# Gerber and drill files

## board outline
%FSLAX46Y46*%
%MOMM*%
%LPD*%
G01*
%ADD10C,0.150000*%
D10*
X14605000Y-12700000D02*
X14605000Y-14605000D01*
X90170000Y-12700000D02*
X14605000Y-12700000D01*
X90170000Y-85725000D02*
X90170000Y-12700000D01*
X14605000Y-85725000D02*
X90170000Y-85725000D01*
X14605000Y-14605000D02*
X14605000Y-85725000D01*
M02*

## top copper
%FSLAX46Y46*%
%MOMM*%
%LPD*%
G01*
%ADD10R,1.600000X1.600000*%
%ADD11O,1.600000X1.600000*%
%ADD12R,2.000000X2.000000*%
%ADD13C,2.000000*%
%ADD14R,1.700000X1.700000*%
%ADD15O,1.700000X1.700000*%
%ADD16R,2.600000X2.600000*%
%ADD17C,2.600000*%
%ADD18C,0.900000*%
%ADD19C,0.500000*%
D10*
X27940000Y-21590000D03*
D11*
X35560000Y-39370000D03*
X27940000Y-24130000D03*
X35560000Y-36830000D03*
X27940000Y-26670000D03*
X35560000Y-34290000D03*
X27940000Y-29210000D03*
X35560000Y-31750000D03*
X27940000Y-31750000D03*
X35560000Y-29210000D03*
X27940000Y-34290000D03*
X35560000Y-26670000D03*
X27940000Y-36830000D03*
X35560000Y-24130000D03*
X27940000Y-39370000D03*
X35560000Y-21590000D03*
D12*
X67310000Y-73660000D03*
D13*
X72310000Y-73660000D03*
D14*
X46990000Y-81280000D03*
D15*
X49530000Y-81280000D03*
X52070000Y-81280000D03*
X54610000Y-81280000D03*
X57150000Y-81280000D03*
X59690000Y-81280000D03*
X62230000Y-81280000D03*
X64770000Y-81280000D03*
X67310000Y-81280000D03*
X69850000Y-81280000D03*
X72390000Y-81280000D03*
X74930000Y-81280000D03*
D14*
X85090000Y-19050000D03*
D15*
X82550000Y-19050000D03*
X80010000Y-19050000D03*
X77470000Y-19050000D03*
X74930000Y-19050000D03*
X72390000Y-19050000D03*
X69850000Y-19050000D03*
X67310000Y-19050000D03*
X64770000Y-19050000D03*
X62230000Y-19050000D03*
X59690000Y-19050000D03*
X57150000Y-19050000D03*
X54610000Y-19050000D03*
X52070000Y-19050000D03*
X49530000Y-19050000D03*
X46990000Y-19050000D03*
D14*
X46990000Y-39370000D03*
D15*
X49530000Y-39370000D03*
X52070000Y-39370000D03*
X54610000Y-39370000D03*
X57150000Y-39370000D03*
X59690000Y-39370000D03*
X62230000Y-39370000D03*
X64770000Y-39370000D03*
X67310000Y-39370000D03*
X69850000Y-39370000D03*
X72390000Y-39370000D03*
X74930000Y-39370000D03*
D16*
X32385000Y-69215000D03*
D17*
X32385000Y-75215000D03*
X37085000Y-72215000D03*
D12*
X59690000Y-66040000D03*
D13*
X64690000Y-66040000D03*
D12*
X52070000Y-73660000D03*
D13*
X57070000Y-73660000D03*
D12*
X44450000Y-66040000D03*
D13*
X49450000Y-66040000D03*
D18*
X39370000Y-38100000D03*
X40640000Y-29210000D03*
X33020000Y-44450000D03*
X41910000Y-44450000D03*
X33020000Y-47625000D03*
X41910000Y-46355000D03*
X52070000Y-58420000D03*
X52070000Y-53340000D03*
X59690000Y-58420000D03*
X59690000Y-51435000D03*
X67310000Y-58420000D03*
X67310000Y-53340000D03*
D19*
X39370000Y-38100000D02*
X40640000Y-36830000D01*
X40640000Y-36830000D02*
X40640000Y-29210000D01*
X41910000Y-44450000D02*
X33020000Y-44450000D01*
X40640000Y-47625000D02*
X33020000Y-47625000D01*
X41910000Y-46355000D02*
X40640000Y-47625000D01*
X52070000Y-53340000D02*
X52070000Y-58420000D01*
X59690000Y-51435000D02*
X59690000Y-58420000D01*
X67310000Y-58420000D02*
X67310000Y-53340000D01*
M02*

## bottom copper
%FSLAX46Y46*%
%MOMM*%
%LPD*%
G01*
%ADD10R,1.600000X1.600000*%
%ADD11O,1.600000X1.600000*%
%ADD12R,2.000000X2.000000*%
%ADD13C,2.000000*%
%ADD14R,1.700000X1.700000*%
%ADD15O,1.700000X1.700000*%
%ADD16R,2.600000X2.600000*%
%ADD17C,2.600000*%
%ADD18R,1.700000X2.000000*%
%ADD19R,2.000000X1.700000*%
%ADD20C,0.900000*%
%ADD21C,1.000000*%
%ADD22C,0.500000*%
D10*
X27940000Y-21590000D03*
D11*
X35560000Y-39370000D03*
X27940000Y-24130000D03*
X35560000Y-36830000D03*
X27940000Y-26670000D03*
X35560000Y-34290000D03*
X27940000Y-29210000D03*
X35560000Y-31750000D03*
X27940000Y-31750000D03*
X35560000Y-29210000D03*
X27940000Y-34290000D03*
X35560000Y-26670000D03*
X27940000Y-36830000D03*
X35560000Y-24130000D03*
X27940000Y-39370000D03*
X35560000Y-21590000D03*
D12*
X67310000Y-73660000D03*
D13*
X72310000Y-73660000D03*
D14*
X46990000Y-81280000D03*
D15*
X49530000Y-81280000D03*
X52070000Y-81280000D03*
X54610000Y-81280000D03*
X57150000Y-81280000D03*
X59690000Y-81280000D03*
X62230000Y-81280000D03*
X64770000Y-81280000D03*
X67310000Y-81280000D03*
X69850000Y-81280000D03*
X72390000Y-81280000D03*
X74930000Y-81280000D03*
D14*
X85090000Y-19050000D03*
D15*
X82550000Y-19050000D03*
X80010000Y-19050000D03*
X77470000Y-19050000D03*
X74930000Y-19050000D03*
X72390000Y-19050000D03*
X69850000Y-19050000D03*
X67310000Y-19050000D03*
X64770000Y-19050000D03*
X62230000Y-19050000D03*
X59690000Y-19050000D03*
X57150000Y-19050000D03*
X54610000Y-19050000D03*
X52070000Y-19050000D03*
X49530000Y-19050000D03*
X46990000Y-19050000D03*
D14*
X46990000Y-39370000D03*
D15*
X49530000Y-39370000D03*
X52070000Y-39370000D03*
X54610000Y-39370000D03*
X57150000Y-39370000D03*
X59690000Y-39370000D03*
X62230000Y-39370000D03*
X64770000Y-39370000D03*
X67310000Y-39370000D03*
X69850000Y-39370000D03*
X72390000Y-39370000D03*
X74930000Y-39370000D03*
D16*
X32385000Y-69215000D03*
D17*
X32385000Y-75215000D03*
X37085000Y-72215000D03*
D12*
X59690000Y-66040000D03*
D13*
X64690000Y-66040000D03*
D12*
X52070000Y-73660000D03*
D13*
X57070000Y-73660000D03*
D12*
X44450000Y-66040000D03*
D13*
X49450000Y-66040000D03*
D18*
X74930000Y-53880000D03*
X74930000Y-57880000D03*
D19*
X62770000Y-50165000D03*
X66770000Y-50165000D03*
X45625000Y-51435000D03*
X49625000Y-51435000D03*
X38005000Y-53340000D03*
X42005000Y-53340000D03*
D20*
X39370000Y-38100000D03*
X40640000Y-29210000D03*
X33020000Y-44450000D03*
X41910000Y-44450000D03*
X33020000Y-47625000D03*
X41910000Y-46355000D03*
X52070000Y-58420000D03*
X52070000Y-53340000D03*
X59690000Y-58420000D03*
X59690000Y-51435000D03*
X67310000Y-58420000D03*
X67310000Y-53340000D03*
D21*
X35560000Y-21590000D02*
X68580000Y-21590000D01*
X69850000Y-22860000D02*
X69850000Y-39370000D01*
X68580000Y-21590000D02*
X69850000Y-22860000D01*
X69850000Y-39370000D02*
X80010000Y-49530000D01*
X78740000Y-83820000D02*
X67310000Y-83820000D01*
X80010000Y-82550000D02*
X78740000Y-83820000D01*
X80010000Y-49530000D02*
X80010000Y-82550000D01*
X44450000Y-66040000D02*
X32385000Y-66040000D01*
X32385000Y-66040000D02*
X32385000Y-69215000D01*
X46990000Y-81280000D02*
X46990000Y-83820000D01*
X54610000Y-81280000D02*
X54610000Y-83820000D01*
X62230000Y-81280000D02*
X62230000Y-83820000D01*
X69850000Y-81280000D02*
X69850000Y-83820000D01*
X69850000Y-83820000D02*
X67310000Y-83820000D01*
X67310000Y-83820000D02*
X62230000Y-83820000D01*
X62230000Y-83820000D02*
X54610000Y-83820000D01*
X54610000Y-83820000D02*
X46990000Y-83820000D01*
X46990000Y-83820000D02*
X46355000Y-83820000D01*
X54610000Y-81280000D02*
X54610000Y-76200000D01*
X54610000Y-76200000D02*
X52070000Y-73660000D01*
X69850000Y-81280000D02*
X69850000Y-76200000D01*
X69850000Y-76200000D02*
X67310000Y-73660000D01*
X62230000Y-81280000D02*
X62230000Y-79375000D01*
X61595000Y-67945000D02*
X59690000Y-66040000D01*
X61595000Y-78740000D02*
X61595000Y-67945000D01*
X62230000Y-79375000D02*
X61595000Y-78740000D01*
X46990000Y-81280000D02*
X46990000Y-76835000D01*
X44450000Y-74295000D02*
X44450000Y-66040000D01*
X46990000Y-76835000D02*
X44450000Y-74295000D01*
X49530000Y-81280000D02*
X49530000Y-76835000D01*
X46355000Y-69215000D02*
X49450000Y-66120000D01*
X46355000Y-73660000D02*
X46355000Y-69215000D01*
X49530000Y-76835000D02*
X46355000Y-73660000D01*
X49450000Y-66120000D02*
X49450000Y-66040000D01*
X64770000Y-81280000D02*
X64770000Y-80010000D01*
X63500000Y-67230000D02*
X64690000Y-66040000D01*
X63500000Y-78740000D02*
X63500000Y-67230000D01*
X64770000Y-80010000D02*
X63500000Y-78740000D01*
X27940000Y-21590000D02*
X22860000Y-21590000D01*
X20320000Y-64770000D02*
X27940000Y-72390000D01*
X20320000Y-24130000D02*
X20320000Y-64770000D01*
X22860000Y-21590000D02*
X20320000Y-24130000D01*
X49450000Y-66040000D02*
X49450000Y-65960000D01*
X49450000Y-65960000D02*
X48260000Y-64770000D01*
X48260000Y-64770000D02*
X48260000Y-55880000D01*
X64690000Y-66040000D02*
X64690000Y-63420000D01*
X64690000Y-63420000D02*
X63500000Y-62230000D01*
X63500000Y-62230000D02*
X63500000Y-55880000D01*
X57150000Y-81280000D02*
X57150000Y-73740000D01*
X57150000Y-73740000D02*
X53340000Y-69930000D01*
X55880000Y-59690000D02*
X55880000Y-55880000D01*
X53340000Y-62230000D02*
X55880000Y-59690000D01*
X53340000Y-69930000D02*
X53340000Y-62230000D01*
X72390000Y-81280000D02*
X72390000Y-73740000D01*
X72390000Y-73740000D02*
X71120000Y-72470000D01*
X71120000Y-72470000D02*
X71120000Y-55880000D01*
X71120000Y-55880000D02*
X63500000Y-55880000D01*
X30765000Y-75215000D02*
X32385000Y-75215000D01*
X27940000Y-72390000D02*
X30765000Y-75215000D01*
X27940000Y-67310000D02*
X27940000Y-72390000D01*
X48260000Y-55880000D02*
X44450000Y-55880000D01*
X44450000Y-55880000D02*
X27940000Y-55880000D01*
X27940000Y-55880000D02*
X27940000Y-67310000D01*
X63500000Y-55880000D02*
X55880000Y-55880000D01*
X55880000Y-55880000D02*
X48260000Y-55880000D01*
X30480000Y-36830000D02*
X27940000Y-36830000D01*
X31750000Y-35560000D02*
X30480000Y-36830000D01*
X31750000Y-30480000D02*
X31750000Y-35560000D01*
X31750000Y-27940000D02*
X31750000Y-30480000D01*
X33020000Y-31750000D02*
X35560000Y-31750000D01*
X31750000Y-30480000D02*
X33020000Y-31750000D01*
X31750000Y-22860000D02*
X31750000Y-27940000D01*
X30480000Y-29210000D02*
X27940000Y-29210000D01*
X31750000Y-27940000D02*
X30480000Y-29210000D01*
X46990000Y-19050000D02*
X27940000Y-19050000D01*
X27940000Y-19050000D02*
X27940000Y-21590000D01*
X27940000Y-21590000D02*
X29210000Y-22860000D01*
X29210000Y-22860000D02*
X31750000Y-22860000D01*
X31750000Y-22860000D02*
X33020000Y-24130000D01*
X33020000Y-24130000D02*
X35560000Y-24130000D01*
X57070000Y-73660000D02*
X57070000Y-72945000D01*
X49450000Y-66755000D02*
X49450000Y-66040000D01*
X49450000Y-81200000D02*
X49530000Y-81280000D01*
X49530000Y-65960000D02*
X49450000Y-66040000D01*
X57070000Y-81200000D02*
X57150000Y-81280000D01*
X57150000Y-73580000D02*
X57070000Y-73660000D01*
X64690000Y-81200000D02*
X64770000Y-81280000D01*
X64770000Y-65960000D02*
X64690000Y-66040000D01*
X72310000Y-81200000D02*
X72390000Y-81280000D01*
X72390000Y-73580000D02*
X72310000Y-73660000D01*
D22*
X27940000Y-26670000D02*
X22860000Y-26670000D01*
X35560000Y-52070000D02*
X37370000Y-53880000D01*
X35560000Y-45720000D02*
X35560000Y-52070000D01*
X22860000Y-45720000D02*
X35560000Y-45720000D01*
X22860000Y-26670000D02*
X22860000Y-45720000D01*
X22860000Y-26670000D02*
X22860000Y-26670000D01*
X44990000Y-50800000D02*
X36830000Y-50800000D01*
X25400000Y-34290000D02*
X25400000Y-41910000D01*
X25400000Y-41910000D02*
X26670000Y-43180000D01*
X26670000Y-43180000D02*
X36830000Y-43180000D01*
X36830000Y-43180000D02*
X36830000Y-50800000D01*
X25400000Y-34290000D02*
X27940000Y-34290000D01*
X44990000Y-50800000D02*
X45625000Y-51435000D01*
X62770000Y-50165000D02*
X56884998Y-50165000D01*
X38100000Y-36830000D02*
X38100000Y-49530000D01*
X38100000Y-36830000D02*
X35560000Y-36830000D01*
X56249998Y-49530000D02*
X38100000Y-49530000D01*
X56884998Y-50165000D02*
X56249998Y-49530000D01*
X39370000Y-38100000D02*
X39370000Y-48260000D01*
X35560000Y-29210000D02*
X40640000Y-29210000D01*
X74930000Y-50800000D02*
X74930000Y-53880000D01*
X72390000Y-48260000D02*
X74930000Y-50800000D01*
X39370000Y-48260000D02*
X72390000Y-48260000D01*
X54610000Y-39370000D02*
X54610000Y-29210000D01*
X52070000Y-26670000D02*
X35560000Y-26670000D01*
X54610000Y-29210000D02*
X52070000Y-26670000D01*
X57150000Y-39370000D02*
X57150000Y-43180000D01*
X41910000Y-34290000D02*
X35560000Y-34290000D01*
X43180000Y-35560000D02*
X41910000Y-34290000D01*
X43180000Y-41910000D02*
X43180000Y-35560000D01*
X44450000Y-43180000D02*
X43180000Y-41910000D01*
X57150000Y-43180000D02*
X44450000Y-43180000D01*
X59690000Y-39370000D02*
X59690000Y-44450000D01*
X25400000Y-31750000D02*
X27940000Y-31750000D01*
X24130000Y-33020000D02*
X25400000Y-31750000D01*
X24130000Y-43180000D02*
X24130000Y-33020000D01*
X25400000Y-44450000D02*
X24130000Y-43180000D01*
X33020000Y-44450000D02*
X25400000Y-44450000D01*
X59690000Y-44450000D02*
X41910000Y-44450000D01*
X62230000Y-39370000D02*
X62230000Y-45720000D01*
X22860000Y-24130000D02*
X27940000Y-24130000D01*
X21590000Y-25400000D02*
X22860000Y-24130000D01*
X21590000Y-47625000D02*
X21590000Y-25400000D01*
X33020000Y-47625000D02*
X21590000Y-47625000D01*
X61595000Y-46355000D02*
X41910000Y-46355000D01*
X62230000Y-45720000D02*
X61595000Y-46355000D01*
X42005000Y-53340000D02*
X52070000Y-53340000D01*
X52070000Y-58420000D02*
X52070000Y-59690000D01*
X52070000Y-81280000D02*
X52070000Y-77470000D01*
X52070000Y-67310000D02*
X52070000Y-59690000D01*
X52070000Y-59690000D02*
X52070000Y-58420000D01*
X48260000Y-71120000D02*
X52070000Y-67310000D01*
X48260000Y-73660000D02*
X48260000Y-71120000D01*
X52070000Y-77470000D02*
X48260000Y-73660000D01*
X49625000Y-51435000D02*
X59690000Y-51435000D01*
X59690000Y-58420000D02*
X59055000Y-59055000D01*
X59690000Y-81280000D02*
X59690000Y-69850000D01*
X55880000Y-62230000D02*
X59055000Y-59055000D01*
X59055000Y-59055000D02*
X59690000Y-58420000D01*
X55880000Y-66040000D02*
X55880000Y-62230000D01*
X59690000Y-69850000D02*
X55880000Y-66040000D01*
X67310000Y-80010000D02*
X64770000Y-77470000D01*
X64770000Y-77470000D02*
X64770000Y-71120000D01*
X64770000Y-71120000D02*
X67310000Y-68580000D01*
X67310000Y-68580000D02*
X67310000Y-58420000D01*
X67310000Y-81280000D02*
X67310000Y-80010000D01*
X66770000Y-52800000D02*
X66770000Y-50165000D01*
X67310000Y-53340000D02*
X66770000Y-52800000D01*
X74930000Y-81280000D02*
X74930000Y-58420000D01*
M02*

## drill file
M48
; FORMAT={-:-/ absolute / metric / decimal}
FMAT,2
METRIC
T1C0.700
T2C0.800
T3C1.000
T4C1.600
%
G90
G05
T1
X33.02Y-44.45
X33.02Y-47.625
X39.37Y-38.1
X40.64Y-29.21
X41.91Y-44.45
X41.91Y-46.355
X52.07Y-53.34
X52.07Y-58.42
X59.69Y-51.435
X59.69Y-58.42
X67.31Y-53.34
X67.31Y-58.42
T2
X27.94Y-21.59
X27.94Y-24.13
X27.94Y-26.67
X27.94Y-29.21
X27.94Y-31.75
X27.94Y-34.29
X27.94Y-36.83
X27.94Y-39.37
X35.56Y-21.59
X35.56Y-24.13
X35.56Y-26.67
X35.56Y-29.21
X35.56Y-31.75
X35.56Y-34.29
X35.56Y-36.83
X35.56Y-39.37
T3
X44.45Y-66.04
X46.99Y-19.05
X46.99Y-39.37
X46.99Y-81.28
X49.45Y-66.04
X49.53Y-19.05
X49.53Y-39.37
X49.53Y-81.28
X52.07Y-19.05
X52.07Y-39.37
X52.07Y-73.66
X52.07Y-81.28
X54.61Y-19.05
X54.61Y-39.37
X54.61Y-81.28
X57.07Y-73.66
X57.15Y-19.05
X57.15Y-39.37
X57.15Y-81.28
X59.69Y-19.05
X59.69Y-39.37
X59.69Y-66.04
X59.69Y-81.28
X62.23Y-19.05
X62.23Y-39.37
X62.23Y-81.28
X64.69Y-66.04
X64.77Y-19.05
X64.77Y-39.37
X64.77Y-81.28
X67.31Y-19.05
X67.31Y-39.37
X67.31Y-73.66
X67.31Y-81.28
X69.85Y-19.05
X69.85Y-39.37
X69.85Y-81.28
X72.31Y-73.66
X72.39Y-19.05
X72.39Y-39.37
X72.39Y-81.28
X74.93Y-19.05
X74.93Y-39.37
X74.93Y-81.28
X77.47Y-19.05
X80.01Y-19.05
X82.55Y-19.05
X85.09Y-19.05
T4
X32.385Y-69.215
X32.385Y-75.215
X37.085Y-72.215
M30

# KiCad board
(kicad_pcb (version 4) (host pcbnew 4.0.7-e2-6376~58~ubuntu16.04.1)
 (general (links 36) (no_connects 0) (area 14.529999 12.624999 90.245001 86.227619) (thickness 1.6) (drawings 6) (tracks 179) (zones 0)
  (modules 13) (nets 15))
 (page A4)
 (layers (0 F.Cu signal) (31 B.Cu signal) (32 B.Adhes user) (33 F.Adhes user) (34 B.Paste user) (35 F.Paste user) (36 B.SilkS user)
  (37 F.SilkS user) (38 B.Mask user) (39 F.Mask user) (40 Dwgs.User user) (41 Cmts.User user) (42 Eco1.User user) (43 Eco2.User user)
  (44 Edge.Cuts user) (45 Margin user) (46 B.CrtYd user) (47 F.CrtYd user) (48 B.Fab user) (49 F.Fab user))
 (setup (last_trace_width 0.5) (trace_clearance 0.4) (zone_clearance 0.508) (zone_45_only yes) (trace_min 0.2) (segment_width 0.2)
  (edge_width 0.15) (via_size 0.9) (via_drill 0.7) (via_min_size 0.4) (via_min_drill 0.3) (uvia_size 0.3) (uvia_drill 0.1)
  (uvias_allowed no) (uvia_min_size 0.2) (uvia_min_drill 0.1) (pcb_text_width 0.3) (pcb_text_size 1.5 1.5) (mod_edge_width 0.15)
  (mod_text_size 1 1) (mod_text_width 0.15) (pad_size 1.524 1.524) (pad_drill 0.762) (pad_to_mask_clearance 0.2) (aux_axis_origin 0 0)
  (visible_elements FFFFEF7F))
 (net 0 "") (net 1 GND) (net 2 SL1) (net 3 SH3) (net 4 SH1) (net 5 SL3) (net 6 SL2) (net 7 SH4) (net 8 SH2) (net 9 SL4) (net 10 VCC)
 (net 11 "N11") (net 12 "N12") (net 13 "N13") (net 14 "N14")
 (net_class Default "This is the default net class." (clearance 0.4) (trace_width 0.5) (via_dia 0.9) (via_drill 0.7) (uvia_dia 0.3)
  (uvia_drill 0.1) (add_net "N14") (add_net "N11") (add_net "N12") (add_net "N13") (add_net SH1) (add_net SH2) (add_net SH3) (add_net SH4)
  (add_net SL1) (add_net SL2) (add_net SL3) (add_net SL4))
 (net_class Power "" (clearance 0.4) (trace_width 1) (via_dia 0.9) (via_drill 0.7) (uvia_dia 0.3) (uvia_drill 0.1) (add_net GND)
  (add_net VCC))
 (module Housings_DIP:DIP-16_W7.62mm (layer F.Cu) (at 27.94 21.59)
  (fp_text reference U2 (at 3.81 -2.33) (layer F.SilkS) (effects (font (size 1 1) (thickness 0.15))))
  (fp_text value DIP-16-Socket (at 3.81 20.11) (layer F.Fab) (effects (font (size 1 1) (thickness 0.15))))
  (pad 1 thru_hole rect (at 0 0) (size 1.6 1.6) (drill 0.8) (layers *.Cu *.Mask) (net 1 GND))
  (pad 9 thru_hole oval (at 7.62 17.78) (size 1.6 1.6) (drill 0.8) (layers *.Cu *.Mask))
  (pad 2 thru_hole oval (at 0 2.54) (size 1.6 1.6) (drill 0.8) (layers *.Cu *.Mask) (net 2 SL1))
  (pad 10 thru_hole oval (at 7.62 15.24) (size 1.6 1.6) (drill 0.8) (layers *.Cu *.Mask) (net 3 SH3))
  (pad 3 thru_hole oval (at 0 5.08) (size 1.6 1.6) (drill 0.8) (layers *.Cu *.Mask) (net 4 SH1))
  (pad 11 thru_hole oval (at 7.62 12.7) (size 1.6 1.6) (drill 0.8) (layers *.Cu *.Mask) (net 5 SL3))
  (pad 4 thru_hole oval (at 0 7.62) (size 1.6 1.6) (drill 0.8) (layers *.Cu *.Mask) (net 1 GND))
  (pad 12 thru_hole oval (at 7.62 10.16) (size 1.6 1.6) (drill 0.8) (layers *.Cu *.Mask) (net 1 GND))
  (pad 5 thru_hole oval (at 0 10.16) (size 1.6 1.6) (drill 0.8) (layers *.Cu *.Mask) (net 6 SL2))
  (pad 13 thru_hole oval (at 7.62 7.62) (size 1.6 1.6) (drill 0.8) (layers *.Cu *.Mask) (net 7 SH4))
  (pad 6 thru_hole oval (at 0 12.7) (size 1.6 1.6) (drill 0.8) (layers *.Cu *.Mask) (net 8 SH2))
  (pad 14 thru_hole oval (at 7.62 5.08) (size 1.6 1.6) (drill 0.8) (layers *.Cu *.Mask) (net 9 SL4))
  (pad 7 thru_hole oval (at 0 15.24) (size 1.6 1.6) (drill 0.8) (layers *.Cu *.Mask) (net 1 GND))
  (pad 15 thru_hole oval (at 7.62 2.54) (size 1.6 1.6) (drill 0.8) (layers *.Cu *.Mask) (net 1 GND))
  (pad 8 thru_hole oval (at 0 17.78) (size 1.6 1.6) (drill 0.8) (layers *.Cu *.Mask))
  (pad 16 thru_hole oval (at 7.62 0) (size 1.6 1.6) (drill 0.8) (layers *.Cu *.Mask) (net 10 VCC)))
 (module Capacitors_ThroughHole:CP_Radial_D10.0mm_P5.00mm (layer F.Cu) (at 67.31 73.66)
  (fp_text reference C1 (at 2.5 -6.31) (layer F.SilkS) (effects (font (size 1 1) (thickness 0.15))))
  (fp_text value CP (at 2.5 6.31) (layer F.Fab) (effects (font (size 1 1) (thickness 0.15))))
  (pad 1 thru_hole rect (at 0 0) (size 2 2) (drill 1) (layers *.Cu *.Mask) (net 10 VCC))
  (pad 2 thru_hole circle (at 5 0) (size 2 2) (drill 1) (layers *.Cu *.Mask) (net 1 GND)))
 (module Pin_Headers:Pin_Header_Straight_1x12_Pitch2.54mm (layer F.Cu) (at 46.99 81.28 90)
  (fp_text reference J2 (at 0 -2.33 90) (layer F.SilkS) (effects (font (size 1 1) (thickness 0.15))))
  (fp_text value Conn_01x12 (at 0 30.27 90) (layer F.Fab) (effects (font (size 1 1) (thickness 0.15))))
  (pad 1 thru_hole rect (at 0 0 90) (size 1.7 1.7) (drill 1) (layers *.Cu *.Mask) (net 10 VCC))
  (pad 2 thru_hole oval (at 0 2.54 90) (size 1.7 1.7) (drill 1) (layers *.Cu *.Mask) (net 1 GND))
  (pad 3 thru_hole oval (at 0 5.08 90) (size 1.7 1.7) (drill 1) (layers *.Cu *.Mask) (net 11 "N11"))
  (pad 4 thru_hole oval (at 0 7.62 90) (size 1.7 1.7) (drill 1) (layers *.Cu *.Mask) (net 10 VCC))
  (pad 5 thru_hole oval (at 0 10.16 90) (size 1.7 1.7) (drill 1) (layers *.Cu *.Mask) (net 1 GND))
  (pad 6 thru_hole oval (at 0 12.7 90) (size 1.7 1.7) (drill 1) (layers *.Cu *.Mask) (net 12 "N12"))
  (pad 7 thru_hole oval (at 0 15.24 90) (size 1.7 1.7) (drill 1) (layers *.Cu *.Mask) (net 10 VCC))
  (pad 8 thru_hole oval (at 0 17.78 90) (size 1.7 1.7) (drill 1) (layers *.Cu *.Mask) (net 1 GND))
  (pad 9 thru_hole oval (at 0 20.32 90) (size 1.7 1.7) (drill 1) (layers *.Cu *.Mask) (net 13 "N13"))
  (pad 10 thru_hole oval (at 0 22.86 90) (size 1.7 1.7) (drill 1) (layers *.Cu *.Mask) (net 10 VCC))
  (pad 11 thru_hole oval (at 0 25.4 90) (size 1.7 1.7) (drill 1) (layers *.Cu *.Mask) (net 1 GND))
  (pad 12 thru_hole oval (at 0 27.94 90) (size 1.7 1.7) (drill 1) (layers *.Cu *.Mask) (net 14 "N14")))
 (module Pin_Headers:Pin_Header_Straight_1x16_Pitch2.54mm (layer F.Cu) (at 85.09 19.05 270)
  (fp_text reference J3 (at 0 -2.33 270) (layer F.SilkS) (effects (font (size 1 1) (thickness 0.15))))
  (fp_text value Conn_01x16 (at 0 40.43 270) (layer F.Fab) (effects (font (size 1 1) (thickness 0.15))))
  (pad 1 thru_hole rect (at 0 0 270) (size 1.7 1.7) (drill 1) (layers *.Cu *.Mask))
  (pad 2 thru_hole oval (at 0 2.54 270) (size 1.7 1.7) (drill 1) (layers *.Cu *.Mask))
  (pad 3 thru_hole oval (at 0 5.08 270) (size 1.7 1.7) (drill 1) (layers *.Cu *.Mask))
  (pad 4 thru_hole oval (at 0 7.62 270) (size 1.7 1.7) (drill 1) (layers *.Cu *.Mask))
  (pad 5 thru_hole oval (at 0 10.16 270) (size 1.7 1.7) (drill 1) (layers *.Cu *.Mask))
  (pad 6 thru_hole oval (at 0 12.7 270) (size 1.7 1.7) (drill 1) (layers *.Cu *.Mask))
  (pad 7 thru_hole oval (at 0 15.24 270) (size 1.7 1.7) (drill 1) (layers *.Cu *.Mask))
  (pad 8 thru_hole oval (at 0 17.78 270) (size 1.7 1.7) (drill 1) (layers *.Cu *.Mask))
  (pad 9 thru_hole oval (at 0 20.32 270) (size 1.7 1.7) (drill 1) (layers *.Cu *.Mask))
  (pad 10 thru_hole oval (at 0 22.86 270) (size 1.7 1.7) (drill 1) (layers *.Cu *.Mask))
  (pad 11 thru_hole oval (at 0 25.4 270) (size 1.7 1.7) (drill 1) (layers *.Cu *.Mask))
  (pad 12 thru_hole oval (at 0 27.94 270) (size 1.7 1.7) (drill 1) (layers *.Cu *.Mask))
  (pad 13 thru_hole oval (at 0 30.48 270) (size 1.7 1.7) (drill 1) (layers *.Cu *.Mask))
  (pad 14 thru_hole oval (at 0 33.02 270) (size 1.7 1.7) (drill 1) (layers *.Cu *.Mask))
  (pad 15 thru_hole oval (at 0 35.56 270) (size 1.7 1.7) (drill 1) (layers *.Cu *.Mask))
  (pad 16 thru_hole oval (at 0 38.1 270) (size 1.7 1.7) (drill 1) (layers *.Cu *.Mask) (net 1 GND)))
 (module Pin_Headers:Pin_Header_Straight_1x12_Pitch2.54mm (layer F.Cu) (at 46.99 39.37 90)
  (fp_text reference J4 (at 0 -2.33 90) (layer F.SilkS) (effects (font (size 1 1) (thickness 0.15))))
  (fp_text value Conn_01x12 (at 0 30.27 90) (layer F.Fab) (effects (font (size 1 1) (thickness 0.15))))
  (pad 1 thru_hole rect (at 0 0 90) (size 1.7 1.7) (drill 1) (layers *.Cu *.Mask))
  (pad 2 thru_hole oval (at 0 2.54 90) (size 1.7 1.7) (drill 1) (layers *.Cu *.Mask))
  (pad 3 thru_hole oval (at 0 5.08 90) (size 1.7 1.7) (drill 1) (layers *.Cu *.Mask))
  (pad 4 thru_hole oval (at 0 7.62 90) (size 1.7 1.7) (drill 1) (layers *.Cu *.Mask) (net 9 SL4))
  (pad 5 thru_hole oval (at 0 10.16 90) (size 1.7 1.7) (drill 1) (layers *.Cu *.Mask) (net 5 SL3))
  (pad 6 thru_hole oval (at 0 12.7 90) (size 1.7 1.7) (drill 1) (layers *.Cu *.Mask) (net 6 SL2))
  (pad 7 thru_hole oval (at 0 15.24 90) (size 1.7 1.7) (drill 1) (layers *.Cu *.Mask) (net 2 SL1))
  (pad 8 thru_hole oval (at 0 17.78 90) (size 1.7 1.7) (drill 1) (layers *.Cu *.Mask))
  (pad 9 thru_hole oval (at 0 20.32 90) (size 1.7 1.7) (drill 1) (layers *.Cu *.Mask))
  (pad 10 thru_hole oval (at 0 22.86 90) (size 1.7 1.7) (drill 1) (layers *.Cu *.Mask) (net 10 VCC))
  (pad 11 thru_hole oval (at 0 25.4 90) (size 1.7 1.7) (drill 1) (layers *.Cu *.Mask))
  (pad 12 thru_hole oval (at 0 27.94 90) (size 1.7 1.7) (drill 1) (layers *.Cu *.Mask)))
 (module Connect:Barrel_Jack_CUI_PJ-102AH (layer F.Cu) (at 32.385 69.215)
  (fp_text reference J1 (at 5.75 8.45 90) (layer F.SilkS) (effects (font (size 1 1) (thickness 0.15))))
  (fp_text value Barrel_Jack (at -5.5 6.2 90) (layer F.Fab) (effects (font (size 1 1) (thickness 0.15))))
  (pad 1 thru_hole rect (at 0 0) (size 2.6 2.6) (drill 1.6) (layers *.Cu *.Mask) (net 10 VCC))
  (pad 2 thru_hole circle (at 0 6) (size 2.6 2.6) (drill 1.6) (layers *.Cu *.Mask) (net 1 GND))
  (pad 3 thru_hole circle (at 4.7 3) (size 2.6 2.6) (drill 1.6) (layers *.Cu *.Mask)))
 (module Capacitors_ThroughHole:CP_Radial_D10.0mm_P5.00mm (layer F.Cu) (at 59.69 66.04)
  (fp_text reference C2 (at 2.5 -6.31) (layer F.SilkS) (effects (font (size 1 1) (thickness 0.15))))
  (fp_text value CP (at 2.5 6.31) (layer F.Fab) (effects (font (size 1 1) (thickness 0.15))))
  (pad 1 thru_hole rect (at 0 0) (size 2 2) (drill 1) (layers *.Cu *.Mask) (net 10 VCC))
  (pad 2 thru_hole circle (at 5 0) (size 2 2) (drill 1) (layers *.Cu *.Mask) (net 1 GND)))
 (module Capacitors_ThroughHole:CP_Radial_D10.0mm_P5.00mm (layer F.Cu) (at 52.07 73.66)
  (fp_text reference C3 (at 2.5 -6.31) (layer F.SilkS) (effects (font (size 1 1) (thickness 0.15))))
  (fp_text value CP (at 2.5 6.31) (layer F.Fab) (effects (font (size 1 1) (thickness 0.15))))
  (pad 1 thru_hole rect (at 0 0) (size 2 2) (drill 1) (layers *.Cu *.Mask) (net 10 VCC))
  (pad 2 thru_hole circle (at 5 0) (size 2 2) (drill 1) (layers *.Cu *.Mask) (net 1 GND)))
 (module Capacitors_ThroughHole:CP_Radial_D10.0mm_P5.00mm (layer F.Cu) (at 44.45 66.04)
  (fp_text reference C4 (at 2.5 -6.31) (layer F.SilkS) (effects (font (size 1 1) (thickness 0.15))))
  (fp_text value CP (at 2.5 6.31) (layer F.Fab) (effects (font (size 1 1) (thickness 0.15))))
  (pad 1 thru_hole rect (at 0 0) (size 2 2) (drill 1) (layers *.Cu *.Mask) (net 10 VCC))
  (pad 2 thru_hole circle (at 5 0) (size 2 2) (drill 1) (layers *.Cu *.Mask) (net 1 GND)))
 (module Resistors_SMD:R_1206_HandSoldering (layer B.Cu) (at 74.93 55.88 270)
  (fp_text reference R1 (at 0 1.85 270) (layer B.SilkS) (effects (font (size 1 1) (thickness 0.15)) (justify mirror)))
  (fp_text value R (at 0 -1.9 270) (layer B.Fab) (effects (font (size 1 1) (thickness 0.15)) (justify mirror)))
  (pad 1 smd rect (at -2 0 270) (size 2 1.7) (layers B.Cu B.Paste B.Mask) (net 7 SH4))
  (pad 2 smd rect (at 2 0 270) (size 2 1.7) (layers B.Cu B.Paste B.Mask) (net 14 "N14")))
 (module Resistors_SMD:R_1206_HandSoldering (layer B.Cu) (at 64.77 50.165)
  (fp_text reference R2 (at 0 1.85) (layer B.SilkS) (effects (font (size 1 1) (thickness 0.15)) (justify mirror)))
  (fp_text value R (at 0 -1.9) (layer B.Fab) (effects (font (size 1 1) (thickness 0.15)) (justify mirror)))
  (pad 1 smd rect (at -2 0) (size 2 1.7) (layers B.Cu B.Paste B.Mask) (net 3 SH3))
  (pad 2 smd rect (at 2 0) (size 2 1.7) (layers B.Cu B.Paste B.Mask) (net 13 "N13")))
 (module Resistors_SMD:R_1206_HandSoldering (layer B.Cu) (at 47.625 51.435)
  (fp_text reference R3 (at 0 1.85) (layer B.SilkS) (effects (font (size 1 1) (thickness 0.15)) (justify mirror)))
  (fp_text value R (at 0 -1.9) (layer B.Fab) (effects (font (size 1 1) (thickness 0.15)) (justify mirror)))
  (pad 1 smd rect (at -2 0) (size 2 1.7) (layers B.Cu B.Paste B.Mask) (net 8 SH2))
  (pad 2 smd rect (at 2 0) (size 2 1.7) (layers B.Cu B.Paste B.Mask) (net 12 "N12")))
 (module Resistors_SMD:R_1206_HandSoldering (layer B.Cu) (at 40.005 53.34)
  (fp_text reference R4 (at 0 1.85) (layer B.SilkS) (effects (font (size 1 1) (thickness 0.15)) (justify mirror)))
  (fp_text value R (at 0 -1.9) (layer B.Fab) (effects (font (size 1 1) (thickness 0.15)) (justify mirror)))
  (pad 1 smd rect (at -2 0) (size 2 1.7) (layers B.Cu B.Paste B.Mask) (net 4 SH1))
  (pad 2 smd rect (at 2 0) (size 2 1.7) (layers B.Cu B.Paste B.Mask) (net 11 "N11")))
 (gr_line (start 14.605 12.7) (end 14.605 14.605) (angle 90) (layer Edge.Cuts) (width 0.15))
 (gr_line (start 90.17 12.7) (end 14.605 12.7) (angle 90) (layer Edge.Cuts) (width 0.15))
 (gr_line (start 90.17 85.725) (end 90.17 12.7) (angle 90) (layer Edge.Cuts) (width 0.15))
 (gr_line (start 14.605 85.725) (end 90.17 85.725) (angle 90) (layer Edge.Cuts) (width 0.15))
 (gr_line (start 14.605 14.605) (end 14.605 85.725) (angle 90) (layer Edge.Cuts) (width 0.15))
 (segment (start 35.56 21.59) (end 68.58 21.59) (width 1) (layer B.Cu) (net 10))
 (segment (start 69.85 22.86) (end 69.85 39.37) (width 1) (layer B.Cu) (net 10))
 (segment (start 68.58 21.59) (end 69.85 22.86) (width 1) (layer B.Cu) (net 10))
 (segment (start 69.85 39.37) (end 80.01 49.53) (width 1) (layer B.Cu) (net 10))
 (segment (start 78.74 83.82) (end 67.31 83.82) (width 1) (layer B.Cu) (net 10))
 (segment (start 80.01 82.55) (end 78.74 83.82) (width 1) (layer B.Cu) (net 10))
 (segment (start 80.01 49.53) (end 80.01 82.55) (width 1) (layer B.Cu) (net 10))
 (segment (start 44.45 66.04) (end 32.385 66.04) (width 1) (layer B.Cu) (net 10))
 (segment (start 32.385 66.04) (end 32.385 69.215) (width 1) (layer B.Cu) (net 10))
 (segment (start 46.99 81.28) (end 46.99 83.82) (width 1) (layer B.Cu) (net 10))
 (segment (start 54.61 81.28) (end 54.61 83.82) (width 1) (layer B.Cu) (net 10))
 (segment (start 62.23 81.28) (end 62.23 83.82) (width 1) (layer B.Cu) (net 10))
 (segment (start 69.85 81.28) (end 69.85 83.82) (width 1) (layer B.Cu) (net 10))
 (segment (start 69.85 83.82) (end 67.31 83.82) (width 1) (layer B.Cu) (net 10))
 (segment (start 67.31 83.82) (end 62.23 83.82) (width 1) (layer B.Cu) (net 10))
 (segment (start 62.23 83.82) (end 54.61 83.82) (width 1) (layer B.Cu) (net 10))
 (segment (start 54.61 83.82) (end 46.99 83.82) (width 1) (layer B.Cu) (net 10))
 (segment (start 46.99 83.82) (end 46.355 83.82) (width 1) (layer B.Cu) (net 10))
 (segment (start 54.61 81.28) (end 54.61 76.2) (width 1) (layer B.Cu) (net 10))
 (segment (start 54.61 76.2) (end 52.07 73.66) (width 1) (layer B.Cu) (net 10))
 (segment (start 69.85 81.28) (end 69.85 76.2) (width 1) (layer B.Cu) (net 10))
 (segment (start 69.85 76.2) (end 67.31 73.66) (width 1) (layer B.Cu) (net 10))
 (segment (start 62.23 81.28) (end 62.23 79.375) (width 1) (layer B.Cu) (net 10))
 (segment (start 61.595 67.945) (end 59.69 66.04) (width 1) (layer B.Cu) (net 10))
 (segment (start 61.595 78.74) (end 61.595 67.945) (width 1) (layer B.Cu) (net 10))
 (segment (start 62.23 79.375) (end 61.595 78.74) (width 1) (layer B.Cu) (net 10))
 (segment (start 46.99 81.28) (end 46.99 76.835) (width 1) (layer B.Cu) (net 10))
 (segment (start 44.45 74.295) (end 44.45 66.04) (width 1) (layer B.Cu) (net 10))
 (segment (start 46.99 76.835) (end 44.45 74.295) (width 1) (layer B.Cu) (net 10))
 (segment (start 49.53 81.28) (end 49.53 76.835) (width 1) (layer B.Cu) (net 1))
 (segment (start 46.355 69.215) (end 49.45 66.12) (width 1) (layer B.Cu) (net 1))
 (segment (start 46.355 73.66) (end 46.355 69.215) (width 1) (layer B.Cu) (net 1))
 (segment (start 49.53 76.835) (end 46.355 73.66) (width 1) (layer B.Cu) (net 1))
 (segment (start 49.45 66.12) (end 49.45 66.04) (width 1) (layer B.Cu) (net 1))
 (segment (start 64.77 81.28) (end 64.77 80.01) (width 1) (layer B.Cu) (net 1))
 (segment (start 63.5 67.23) (end 64.69 66.04) (width 1) (layer B.Cu) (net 1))
 (segment (start 63.5 78.74) (end 63.5 67.23) (width 1) (layer B.Cu) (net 1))
 (segment (start 64.77 80.01) (end 63.5 78.74) (width 1) (layer B.Cu) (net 1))
 (segment (start 27.94 21.59) (end 22.86 21.59) (width 1) (layer B.Cu) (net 1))
 (segment (start 20.32 64.77) (end 27.94 72.39) (width 1) (layer B.Cu) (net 1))
 (segment (start 20.32 24.13) (end 20.32 64.77) (width 1) (layer B.Cu) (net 1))
 (segment (start 22.86 21.59) (end 20.32 24.13) (width 1) (layer B.Cu) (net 1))
 (segment (start 49.45 66.04) (end 49.45 65.96) (width 1) (layer B.Cu) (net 1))
 (segment (start 49.45 65.96) (end 48.26 64.77) (width 1) (layer B.Cu) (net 1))
 (segment (start 48.26 64.77) (end 48.26 55.88) (width 1) (layer B.Cu) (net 1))
 (segment (start 64.69 66.04) (end 64.69 63.42) (width 1) (layer B.Cu) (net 1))
 (segment (start 64.69 63.42) (end 63.5 62.23) (width 1) (layer B.Cu) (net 1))
 (segment (start 63.5 62.23) (end 63.5 55.88) (width 1) (layer B.Cu) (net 1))
 (segment (start 57.15 81.28) (end 57.15 73.74) (width 1) (layer B.Cu) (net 1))
 (segment (start 57.15 73.74) (end 53.34 69.93) (width 1) (layer B.Cu) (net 1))
 (segment (start 55.88 59.69) (end 55.88 55.88) (width 1) (layer B.Cu) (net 1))
 (segment (start 53.34 62.23) (end 55.88 59.69) (width 1) (layer B.Cu) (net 1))
 (segment (start 53.34 69.93) (end 53.34 62.23) (width 1) (layer B.Cu) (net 1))
 (segment (start 72.39 81.28) (end 72.39 73.74) (width 1) (layer B.Cu) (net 1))
 (segment (start 72.39 73.74) (end 71.12 72.47) (width 1) (layer B.Cu) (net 1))
 (segment (start 71.12 72.47) (end 71.12 55.88) (width 1) (layer B.Cu) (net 1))
 (segment (start 71.12 55.88) (end 63.5 55.88) (width 1) (layer B.Cu) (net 1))
 (segment (start 30.765 75.215) (end 32.385 75.215) (width 1) (layer B.Cu) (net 1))
 (segment (start 27.94 72.39) (end 30.765 75.215) (width 1) (layer B.Cu) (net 1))
 (segment (start 27.94 67.31) (end 27.94 72.39) (width 1) (layer B.Cu) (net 1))
 (segment (start 48.26 55.88) (end 44.45 55.88) (width 1) (layer B.Cu) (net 1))
 (segment (start 44.45 55.88) (end 27.94 55.88) (width 1) (layer B.Cu) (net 1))
 (segment (start 27.94 55.88) (end 27.94 67.31) (width 1) (layer B.Cu) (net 1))
 (segment (start 63.5 55.88) (end 55.88 55.88) (width 1) (layer B.Cu) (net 1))
 (segment (start 55.88 55.88) (end 48.26 55.88) (width 1) (layer B.Cu) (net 1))
 (segment (start 30.48 36.83) (end 27.94 36.83) (width 1) (layer B.Cu) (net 1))
 (segment (start 31.75 35.56) (end 30.48 36.83) (width 1) (layer B.Cu) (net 1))
 (segment (start 31.75 30.48) (end 31.75 35.56) (width 1) (layer B.Cu) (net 1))
 (segment (start 31.75 27.94) (end 31.75 30.48) (width 1) (layer B.Cu) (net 1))
 (segment (start 33.02 31.75) (end 35.56 31.75) (width 1) (layer B.Cu) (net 1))
 (segment (start 31.75 30.48) (end 33.02 31.75) (width 1) (layer B.Cu) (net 1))
 (segment (start 31.75 22.86) (end 31.75 27.94) (width 1) (layer B.Cu) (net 1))
 (segment (start 30.48 29.21) (end 27.94 29.21) (width 1) (layer B.Cu) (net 1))
 (segment (start 31.75 27.94) (end 30.48 29.21) (width 1) (layer B.Cu) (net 1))
 (segment (start 46.99 19.05) (end 27.94 19.05) (width 1) (layer B.Cu) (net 1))
 (segment (start 27.94 19.05) (end 27.94 21.59) (width 1) (layer B.Cu) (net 1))
 (segment (start 27.94 21.59) (end 29.21 22.86) (width 1) (layer B.Cu) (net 1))
 (segment (start 29.21 22.86) (end 31.75 22.86) (width 1) (layer B.Cu) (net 1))
 (segment (start 31.75 22.86) (end 33.02 24.13) (width 1) (layer B.Cu) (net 1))
 (segment (start 33.02 24.13) (end 35.56 24.13) (width 1) (layer B.Cu) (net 1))
 (segment (start 57.07 73.66) (end 57.07 72.945) (width 1) (layer B.Cu) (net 1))
 (segment (start 49.45 66.755) (end 49.45 66.04) (width 1) (layer B.Cu) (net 1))
 (segment (start 49.45 81.2) (end 49.53 81.28) (width 1) (layer B.Cu) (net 1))
 (segment (start 49.53 65.96) (end 49.45 66.04) (width 1) (layer B.Cu) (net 1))
 (segment (start 57.07 81.2) (end 57.15 81.28) (width 1) (layer B.Cu) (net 1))
 (segment (start 57.15 73.58) (end 57.07 73.66) (width 1) (layer B.Cu) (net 1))
 (segment (start 64.69 81.2) (end 64.77 81.28) (width 1) (layer B.Cu) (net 1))
 (segment (start 64.77 65.96) (end 64.69 66.04) (width 1) (layer B.Cu) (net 1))
 (segment (start 72.31 81.2) (end 72.39 81.28) (width 1) (layer B.Cu) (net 1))
 (segment (start 72.39 73.58) (end 72.31 73.66) (width 1) (layer B.Cu) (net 1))
 (segment (start 27.94 26.67) (end 22.86 26.67) (width 0.5) (layer B.Cu) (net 4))
 (segment (start 35.56 52.07) (end 37.37 53.88) (width 0.5) (layer B.Cu) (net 4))
 (segment (start 35.56 45.72) (end 35.56 52.07) (width 0.5) (layer B.Cu) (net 4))
 (segment (start 22.86 45.72) (end 35.56 45.72) (width 0.5) (layer B.Cu) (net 4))
 (segment (start 22.86 26.67) (end 22.86 45.72) (width 0.5) (layer B.Cu) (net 4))
 (segment (start 22.86 26.67) (end 22.86 26.67) (width 0.5) (layer B.Cu) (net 4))
 (segment (start 44.99 50.8) (end 36.83 50.8) (width 0.5) (layer B.Cu) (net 8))
 (segment (start 25.4 34.29) (end 25.4 41.91) (width 0.5) (layer B.Cu) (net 8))
 (segment (start 25.4 41.91) (end 26.67 43.18) (width 0.5) (layer B.Cu) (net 8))
 (segment (start 26.67 43.18) (end 36.83 43.18) (width 0.5) (layer B.Cu) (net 8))
 (segment (start 36.83 43.18) (end 36.83 50.8) (width 0.5) (layer B.Cu) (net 8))
 (segment (start 25.4 34.29) (end 27.94 34.29) (width 0.5) (layer B.Cu) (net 8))
 (segment (start 44.99 50.8) (end 45.625 51.435) (width 0.5) (layer B.Cu) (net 8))
 (segment (start 62.77 50.165) (end 56.884998 50.165) (width 0.5) (layer B.Cu) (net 3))
 (segment (start 38.1 36.83) (end 38.1 49.53) (width 0.5) (layer B.Cu) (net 3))
 (segment (start 38.1 36.83) (end 35.56 36.83) (width 0.5) (layer B.Cu) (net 3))
 (segment (start 56.249998 49.53) (end 38.1 49.53) (width 0.5) (layer B.Cu) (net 3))
 (segment (start 56.884998 50.165) (end 56.249998 49.53) (width 0.5) (layer B.Cu) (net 3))
 (segment (start 39.37 38.1) (end 39.37 48.26) (width 0.5) (layer B.Cu) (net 7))
 (via (at 39.37 38.1) (size 0.9) (drill 0.7) (layers F.Cu B.Cu) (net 7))
 (segment (start 39.37 38.1) (end 40.64 36.83) (width 0.5) (layer F.Cu) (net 7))
 (segment (start 40.64 36.83) (end 40.64 29.21) (width 0.5) (layer F.Cu) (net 7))
 (via (at 40.64 29.21) (size 0.9) (drill 0.7) (layers F.Cu B.Cu) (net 7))
 (segment (start 35.56 29.21) (end 40.64 29.21) (width 0.5) (layer B.Cu) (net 7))
 (segment (start 74.93 50.8) (end 74.93 53.88) (width 0.5) (layer B.Cu) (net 7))
 (segment (start 72.39 48.26) (end 74.93 50.8) (width 0.5) (layer B.Cu) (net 7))
 (segment (start 39.37 48.26) (end 72.39 48.26) (width 0.5) (layer B.Cu) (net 7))
 (segment (start 54.61 39.37) (end 54.61 29.21) (width 0.5) (layer B.Cu) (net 9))
 (segment (start 52.07 26.67) (end 35.56 26.67) (width 0.5) (layer B.Cu) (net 9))
 (segment (start 54.61 29.21) (end 52.07 26.67) (width 0.5) (layer B.Cu) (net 9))
 (segment (start 57.15 39.37) (end 57.15 43.18) (width 0.5) (layer B.Cu) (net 5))
 (segment (start 41.91 34.29) (end 35.56 34.29) (width 0.5) (layer B.Cu) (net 5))
 (segment (start 43.18 35.56) (end 41.91 34.29) (width 0.5) (layer B.Cu) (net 5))
 (segment (start 43.18 41.91) (end 43.18 35.56) (width 0.5) (layer B.Cu) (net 5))
 (segment (start 44.45 43.18) (end 43.18 41.91) (width 0.5) (layer B.Cu) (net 5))
 (segment (start 57.15 43.18) (end 44.45 43.18) (width 0.5) (layer B.Cu) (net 5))
 (segment (start 59.69 39.37) (end 59.69 44.45) (width 0.5) (layer B.Cu) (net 6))
 (segment (start 25.4 31.75) (end 27.94 31.75) (width 0.5) (layer B.Cu) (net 6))
 (segment (start 24.13 33.02) (end 25.4 31.75) (width 0.5) (layer B.Cu) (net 6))
 (segment (start 24.13 43.18) (end 24.13 33.02) (width 0.5) (layer B.Cu) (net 6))
 (segment (start 25.4 44.45) (end 24.13 43.18) (width 0.5) (layer B.Cu) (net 6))
 (segment (start 33.02 44.45) (end 25.4 44.45) (width 0.5) (layer B.Cu) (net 6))
 (via (at 33.02 44.45) (size 0.9) (drill 0.7) (layers F.Cu B.Cu) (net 6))
 (segment (start 41.91 44.45) (end 33.02 44.45) (width 0.5) (layer F.Cu) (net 6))
 (via (at 41.91 44.45) (size 0.9) (drill 0.7) (layers F.Cu B.Cu) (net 6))
 (segment (start 59.69 44.45) (end 41.91 44.45) (width 0.5) (layer B.Cu) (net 6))
 (segment (start 62.23 39.37) (end 62.23 45.72) (width 0.5) (layer B.Cu) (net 2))
 (segment (start 22.86 24.13) (end 27.94 24.13) (width 0.5) (layer B.Cu) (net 2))
 (segment (start 21.59 25.4) (end 22.86 24.13) (width 0.5) (layer B.Cu) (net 2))
 (segment (start 21.59 47.625) (end 21.59 25.4) (width 0.5) (layer B.Cu) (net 2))
 (segment (start 33.02 47.625) (end 21.59 47.625) (width 0.5) (layer B.Cu) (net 2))
 (via (at 33.02 47.625) (size 0.9) (drill 0.7) (layers F.Cu B.Cu) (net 2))
 (segment (start 40.64 47.625) (end 33.02 47.625) (width 0.5) (layer F.Cu) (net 2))
 (segment (start 41.91 46.355) (end 40.64 47.625) (width 0.5) (layer F.Cu) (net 2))
 (via (at 41.91 46.355) (size 0.9) (drill 0.7) (layers F.Cu B.Cu) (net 2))
 (segment (start 61.595 46.355) (end 41.91 46.355) (width 0.5) (layer B.Cu) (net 2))
 (segment (start 62.23 45.72) (end 61.595 46.355) (width 0.5) (layer B.Cu) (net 2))
 (segment (start 42.005 53.34) (end 52.07 53.34) (width 0.5) (layer B.Cu) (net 11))
 (via (at 52.07 58.42) (size 0.9) (drill 0.7) (layers F.Cu B.Cu) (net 11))
 (segment (start 52.07 53.34) (end 52.07 58.42) (width 0.5) (layer F.Cu) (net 11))
 (via (at 52.07 53.34) (size 0.9) (drill 0.7) (layers F.Cu B.Cu) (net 11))
 (segment (start 52.07 58.42) (end 52.07 59.69) (width 0.5) (layer B.Cu) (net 11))
 (segment (start 52.07 81.28) (end 52.07 77.47) (width 0.5) (layer B.Cu) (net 11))
 (segment (start 52.07 67.31) (end 52.07 59.69) (width 0.5) (layer B.Cu) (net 11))
 (segment (start 52.07 59.69) (end 52.07 58.42) (width 0.5) (layer B.Cu) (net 11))
 (segment (start 48.26 71.12) (end 52.07 67.31) (width 0.5) (layer B.Cu) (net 11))
 (segment (start 48.26 73.66) (end 48.26 71.12) (width 0.5) (layer B.Cu) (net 11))
 (segment (start 52.07 77.47) (end 48.26 73.66) (width 0.5) (layer B.Cu) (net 11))
 (segment (start 49.625 51.435) (end 59.69 51.435) (width 0.5) (layer B.Cu) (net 12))
 (via (at 59.69 58.42) (size 0.9) (drill 0.7) (layers F.Cu B.Cu) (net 12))
 (segment (start 59.69 51.435) (end 59.69 58.42) (width 0.5) (layer F.Cu) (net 12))
 (via (at 59.69 51.435) (size 0.9) (drill 0.7) (layers F.Cu B.Cu) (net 12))
 (segment (start 59.69 58.42) (end 59.055 59.055) (width 0.5) (layer B.Cu) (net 12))
 (segment (start 59.69 81.28) (end 59.69 69.85) (width 0.5) (layer B.Cu) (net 12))
 (segment (start 55.88 62.23) (end 59.055 59.055) (width 0.5) (layer B.Cu) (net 12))
 (segment (start 59.055 59.055) (end 59.69 58.42) (width 0.5) (layer B.Cu) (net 12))
 (segment (start 55.88 66.04) (end 55.88 62.23) (width 0.5) (layer B.Cu) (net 12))
 (segment (start 59.69 69.85) (end 55.88 66.04) (width 0.5) (layer B.Cu) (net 12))
 (via (at 67.31 58.42) (size 0.9) (drill 0.7) (layers F.Cu B.Cu) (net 13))
 (segment (start 67.31 80.01) (end 64.77 77.47) (width 0.5) (layer B.Cu) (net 13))
 (segment (start 64.77 77.47) (end 64.77 71.12) (width 0.5) (layer B.Cu) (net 13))
 (segment (start 64.77 71.12) (end 67.31 68.58) (width 0.5) (layer B.Cu) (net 13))
 (segment (start 67.31 68.58) (end 67.31 58.42) (width 0.5) (layer B.Cu) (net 13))
 (segment (start 67.31 81.28) (end 67.31 80.01) (width 0.5) (layer B.Cu) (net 13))
 (segment (start 66.77 52.8) (end 66.77 50.165) (width 0.5) (layer B.Cu) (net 13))
 (segment (start 67.31 53.34) (end 66.77 52.8) (width 0.5) (layer B.Cu) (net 13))
 (via (at 67.31 53.34) (size 0.9) (drill 0.7) (layers F.Cu B.Cu) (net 13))
 (segment (start 67.31 58.42) (end 67.31 53.34) (width 0.5) (layer F.Cu) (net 13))
 (segment (start 74.93 81.28) (end 74.93 58.42) (width 0.5) (layer B.Cu) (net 14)))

